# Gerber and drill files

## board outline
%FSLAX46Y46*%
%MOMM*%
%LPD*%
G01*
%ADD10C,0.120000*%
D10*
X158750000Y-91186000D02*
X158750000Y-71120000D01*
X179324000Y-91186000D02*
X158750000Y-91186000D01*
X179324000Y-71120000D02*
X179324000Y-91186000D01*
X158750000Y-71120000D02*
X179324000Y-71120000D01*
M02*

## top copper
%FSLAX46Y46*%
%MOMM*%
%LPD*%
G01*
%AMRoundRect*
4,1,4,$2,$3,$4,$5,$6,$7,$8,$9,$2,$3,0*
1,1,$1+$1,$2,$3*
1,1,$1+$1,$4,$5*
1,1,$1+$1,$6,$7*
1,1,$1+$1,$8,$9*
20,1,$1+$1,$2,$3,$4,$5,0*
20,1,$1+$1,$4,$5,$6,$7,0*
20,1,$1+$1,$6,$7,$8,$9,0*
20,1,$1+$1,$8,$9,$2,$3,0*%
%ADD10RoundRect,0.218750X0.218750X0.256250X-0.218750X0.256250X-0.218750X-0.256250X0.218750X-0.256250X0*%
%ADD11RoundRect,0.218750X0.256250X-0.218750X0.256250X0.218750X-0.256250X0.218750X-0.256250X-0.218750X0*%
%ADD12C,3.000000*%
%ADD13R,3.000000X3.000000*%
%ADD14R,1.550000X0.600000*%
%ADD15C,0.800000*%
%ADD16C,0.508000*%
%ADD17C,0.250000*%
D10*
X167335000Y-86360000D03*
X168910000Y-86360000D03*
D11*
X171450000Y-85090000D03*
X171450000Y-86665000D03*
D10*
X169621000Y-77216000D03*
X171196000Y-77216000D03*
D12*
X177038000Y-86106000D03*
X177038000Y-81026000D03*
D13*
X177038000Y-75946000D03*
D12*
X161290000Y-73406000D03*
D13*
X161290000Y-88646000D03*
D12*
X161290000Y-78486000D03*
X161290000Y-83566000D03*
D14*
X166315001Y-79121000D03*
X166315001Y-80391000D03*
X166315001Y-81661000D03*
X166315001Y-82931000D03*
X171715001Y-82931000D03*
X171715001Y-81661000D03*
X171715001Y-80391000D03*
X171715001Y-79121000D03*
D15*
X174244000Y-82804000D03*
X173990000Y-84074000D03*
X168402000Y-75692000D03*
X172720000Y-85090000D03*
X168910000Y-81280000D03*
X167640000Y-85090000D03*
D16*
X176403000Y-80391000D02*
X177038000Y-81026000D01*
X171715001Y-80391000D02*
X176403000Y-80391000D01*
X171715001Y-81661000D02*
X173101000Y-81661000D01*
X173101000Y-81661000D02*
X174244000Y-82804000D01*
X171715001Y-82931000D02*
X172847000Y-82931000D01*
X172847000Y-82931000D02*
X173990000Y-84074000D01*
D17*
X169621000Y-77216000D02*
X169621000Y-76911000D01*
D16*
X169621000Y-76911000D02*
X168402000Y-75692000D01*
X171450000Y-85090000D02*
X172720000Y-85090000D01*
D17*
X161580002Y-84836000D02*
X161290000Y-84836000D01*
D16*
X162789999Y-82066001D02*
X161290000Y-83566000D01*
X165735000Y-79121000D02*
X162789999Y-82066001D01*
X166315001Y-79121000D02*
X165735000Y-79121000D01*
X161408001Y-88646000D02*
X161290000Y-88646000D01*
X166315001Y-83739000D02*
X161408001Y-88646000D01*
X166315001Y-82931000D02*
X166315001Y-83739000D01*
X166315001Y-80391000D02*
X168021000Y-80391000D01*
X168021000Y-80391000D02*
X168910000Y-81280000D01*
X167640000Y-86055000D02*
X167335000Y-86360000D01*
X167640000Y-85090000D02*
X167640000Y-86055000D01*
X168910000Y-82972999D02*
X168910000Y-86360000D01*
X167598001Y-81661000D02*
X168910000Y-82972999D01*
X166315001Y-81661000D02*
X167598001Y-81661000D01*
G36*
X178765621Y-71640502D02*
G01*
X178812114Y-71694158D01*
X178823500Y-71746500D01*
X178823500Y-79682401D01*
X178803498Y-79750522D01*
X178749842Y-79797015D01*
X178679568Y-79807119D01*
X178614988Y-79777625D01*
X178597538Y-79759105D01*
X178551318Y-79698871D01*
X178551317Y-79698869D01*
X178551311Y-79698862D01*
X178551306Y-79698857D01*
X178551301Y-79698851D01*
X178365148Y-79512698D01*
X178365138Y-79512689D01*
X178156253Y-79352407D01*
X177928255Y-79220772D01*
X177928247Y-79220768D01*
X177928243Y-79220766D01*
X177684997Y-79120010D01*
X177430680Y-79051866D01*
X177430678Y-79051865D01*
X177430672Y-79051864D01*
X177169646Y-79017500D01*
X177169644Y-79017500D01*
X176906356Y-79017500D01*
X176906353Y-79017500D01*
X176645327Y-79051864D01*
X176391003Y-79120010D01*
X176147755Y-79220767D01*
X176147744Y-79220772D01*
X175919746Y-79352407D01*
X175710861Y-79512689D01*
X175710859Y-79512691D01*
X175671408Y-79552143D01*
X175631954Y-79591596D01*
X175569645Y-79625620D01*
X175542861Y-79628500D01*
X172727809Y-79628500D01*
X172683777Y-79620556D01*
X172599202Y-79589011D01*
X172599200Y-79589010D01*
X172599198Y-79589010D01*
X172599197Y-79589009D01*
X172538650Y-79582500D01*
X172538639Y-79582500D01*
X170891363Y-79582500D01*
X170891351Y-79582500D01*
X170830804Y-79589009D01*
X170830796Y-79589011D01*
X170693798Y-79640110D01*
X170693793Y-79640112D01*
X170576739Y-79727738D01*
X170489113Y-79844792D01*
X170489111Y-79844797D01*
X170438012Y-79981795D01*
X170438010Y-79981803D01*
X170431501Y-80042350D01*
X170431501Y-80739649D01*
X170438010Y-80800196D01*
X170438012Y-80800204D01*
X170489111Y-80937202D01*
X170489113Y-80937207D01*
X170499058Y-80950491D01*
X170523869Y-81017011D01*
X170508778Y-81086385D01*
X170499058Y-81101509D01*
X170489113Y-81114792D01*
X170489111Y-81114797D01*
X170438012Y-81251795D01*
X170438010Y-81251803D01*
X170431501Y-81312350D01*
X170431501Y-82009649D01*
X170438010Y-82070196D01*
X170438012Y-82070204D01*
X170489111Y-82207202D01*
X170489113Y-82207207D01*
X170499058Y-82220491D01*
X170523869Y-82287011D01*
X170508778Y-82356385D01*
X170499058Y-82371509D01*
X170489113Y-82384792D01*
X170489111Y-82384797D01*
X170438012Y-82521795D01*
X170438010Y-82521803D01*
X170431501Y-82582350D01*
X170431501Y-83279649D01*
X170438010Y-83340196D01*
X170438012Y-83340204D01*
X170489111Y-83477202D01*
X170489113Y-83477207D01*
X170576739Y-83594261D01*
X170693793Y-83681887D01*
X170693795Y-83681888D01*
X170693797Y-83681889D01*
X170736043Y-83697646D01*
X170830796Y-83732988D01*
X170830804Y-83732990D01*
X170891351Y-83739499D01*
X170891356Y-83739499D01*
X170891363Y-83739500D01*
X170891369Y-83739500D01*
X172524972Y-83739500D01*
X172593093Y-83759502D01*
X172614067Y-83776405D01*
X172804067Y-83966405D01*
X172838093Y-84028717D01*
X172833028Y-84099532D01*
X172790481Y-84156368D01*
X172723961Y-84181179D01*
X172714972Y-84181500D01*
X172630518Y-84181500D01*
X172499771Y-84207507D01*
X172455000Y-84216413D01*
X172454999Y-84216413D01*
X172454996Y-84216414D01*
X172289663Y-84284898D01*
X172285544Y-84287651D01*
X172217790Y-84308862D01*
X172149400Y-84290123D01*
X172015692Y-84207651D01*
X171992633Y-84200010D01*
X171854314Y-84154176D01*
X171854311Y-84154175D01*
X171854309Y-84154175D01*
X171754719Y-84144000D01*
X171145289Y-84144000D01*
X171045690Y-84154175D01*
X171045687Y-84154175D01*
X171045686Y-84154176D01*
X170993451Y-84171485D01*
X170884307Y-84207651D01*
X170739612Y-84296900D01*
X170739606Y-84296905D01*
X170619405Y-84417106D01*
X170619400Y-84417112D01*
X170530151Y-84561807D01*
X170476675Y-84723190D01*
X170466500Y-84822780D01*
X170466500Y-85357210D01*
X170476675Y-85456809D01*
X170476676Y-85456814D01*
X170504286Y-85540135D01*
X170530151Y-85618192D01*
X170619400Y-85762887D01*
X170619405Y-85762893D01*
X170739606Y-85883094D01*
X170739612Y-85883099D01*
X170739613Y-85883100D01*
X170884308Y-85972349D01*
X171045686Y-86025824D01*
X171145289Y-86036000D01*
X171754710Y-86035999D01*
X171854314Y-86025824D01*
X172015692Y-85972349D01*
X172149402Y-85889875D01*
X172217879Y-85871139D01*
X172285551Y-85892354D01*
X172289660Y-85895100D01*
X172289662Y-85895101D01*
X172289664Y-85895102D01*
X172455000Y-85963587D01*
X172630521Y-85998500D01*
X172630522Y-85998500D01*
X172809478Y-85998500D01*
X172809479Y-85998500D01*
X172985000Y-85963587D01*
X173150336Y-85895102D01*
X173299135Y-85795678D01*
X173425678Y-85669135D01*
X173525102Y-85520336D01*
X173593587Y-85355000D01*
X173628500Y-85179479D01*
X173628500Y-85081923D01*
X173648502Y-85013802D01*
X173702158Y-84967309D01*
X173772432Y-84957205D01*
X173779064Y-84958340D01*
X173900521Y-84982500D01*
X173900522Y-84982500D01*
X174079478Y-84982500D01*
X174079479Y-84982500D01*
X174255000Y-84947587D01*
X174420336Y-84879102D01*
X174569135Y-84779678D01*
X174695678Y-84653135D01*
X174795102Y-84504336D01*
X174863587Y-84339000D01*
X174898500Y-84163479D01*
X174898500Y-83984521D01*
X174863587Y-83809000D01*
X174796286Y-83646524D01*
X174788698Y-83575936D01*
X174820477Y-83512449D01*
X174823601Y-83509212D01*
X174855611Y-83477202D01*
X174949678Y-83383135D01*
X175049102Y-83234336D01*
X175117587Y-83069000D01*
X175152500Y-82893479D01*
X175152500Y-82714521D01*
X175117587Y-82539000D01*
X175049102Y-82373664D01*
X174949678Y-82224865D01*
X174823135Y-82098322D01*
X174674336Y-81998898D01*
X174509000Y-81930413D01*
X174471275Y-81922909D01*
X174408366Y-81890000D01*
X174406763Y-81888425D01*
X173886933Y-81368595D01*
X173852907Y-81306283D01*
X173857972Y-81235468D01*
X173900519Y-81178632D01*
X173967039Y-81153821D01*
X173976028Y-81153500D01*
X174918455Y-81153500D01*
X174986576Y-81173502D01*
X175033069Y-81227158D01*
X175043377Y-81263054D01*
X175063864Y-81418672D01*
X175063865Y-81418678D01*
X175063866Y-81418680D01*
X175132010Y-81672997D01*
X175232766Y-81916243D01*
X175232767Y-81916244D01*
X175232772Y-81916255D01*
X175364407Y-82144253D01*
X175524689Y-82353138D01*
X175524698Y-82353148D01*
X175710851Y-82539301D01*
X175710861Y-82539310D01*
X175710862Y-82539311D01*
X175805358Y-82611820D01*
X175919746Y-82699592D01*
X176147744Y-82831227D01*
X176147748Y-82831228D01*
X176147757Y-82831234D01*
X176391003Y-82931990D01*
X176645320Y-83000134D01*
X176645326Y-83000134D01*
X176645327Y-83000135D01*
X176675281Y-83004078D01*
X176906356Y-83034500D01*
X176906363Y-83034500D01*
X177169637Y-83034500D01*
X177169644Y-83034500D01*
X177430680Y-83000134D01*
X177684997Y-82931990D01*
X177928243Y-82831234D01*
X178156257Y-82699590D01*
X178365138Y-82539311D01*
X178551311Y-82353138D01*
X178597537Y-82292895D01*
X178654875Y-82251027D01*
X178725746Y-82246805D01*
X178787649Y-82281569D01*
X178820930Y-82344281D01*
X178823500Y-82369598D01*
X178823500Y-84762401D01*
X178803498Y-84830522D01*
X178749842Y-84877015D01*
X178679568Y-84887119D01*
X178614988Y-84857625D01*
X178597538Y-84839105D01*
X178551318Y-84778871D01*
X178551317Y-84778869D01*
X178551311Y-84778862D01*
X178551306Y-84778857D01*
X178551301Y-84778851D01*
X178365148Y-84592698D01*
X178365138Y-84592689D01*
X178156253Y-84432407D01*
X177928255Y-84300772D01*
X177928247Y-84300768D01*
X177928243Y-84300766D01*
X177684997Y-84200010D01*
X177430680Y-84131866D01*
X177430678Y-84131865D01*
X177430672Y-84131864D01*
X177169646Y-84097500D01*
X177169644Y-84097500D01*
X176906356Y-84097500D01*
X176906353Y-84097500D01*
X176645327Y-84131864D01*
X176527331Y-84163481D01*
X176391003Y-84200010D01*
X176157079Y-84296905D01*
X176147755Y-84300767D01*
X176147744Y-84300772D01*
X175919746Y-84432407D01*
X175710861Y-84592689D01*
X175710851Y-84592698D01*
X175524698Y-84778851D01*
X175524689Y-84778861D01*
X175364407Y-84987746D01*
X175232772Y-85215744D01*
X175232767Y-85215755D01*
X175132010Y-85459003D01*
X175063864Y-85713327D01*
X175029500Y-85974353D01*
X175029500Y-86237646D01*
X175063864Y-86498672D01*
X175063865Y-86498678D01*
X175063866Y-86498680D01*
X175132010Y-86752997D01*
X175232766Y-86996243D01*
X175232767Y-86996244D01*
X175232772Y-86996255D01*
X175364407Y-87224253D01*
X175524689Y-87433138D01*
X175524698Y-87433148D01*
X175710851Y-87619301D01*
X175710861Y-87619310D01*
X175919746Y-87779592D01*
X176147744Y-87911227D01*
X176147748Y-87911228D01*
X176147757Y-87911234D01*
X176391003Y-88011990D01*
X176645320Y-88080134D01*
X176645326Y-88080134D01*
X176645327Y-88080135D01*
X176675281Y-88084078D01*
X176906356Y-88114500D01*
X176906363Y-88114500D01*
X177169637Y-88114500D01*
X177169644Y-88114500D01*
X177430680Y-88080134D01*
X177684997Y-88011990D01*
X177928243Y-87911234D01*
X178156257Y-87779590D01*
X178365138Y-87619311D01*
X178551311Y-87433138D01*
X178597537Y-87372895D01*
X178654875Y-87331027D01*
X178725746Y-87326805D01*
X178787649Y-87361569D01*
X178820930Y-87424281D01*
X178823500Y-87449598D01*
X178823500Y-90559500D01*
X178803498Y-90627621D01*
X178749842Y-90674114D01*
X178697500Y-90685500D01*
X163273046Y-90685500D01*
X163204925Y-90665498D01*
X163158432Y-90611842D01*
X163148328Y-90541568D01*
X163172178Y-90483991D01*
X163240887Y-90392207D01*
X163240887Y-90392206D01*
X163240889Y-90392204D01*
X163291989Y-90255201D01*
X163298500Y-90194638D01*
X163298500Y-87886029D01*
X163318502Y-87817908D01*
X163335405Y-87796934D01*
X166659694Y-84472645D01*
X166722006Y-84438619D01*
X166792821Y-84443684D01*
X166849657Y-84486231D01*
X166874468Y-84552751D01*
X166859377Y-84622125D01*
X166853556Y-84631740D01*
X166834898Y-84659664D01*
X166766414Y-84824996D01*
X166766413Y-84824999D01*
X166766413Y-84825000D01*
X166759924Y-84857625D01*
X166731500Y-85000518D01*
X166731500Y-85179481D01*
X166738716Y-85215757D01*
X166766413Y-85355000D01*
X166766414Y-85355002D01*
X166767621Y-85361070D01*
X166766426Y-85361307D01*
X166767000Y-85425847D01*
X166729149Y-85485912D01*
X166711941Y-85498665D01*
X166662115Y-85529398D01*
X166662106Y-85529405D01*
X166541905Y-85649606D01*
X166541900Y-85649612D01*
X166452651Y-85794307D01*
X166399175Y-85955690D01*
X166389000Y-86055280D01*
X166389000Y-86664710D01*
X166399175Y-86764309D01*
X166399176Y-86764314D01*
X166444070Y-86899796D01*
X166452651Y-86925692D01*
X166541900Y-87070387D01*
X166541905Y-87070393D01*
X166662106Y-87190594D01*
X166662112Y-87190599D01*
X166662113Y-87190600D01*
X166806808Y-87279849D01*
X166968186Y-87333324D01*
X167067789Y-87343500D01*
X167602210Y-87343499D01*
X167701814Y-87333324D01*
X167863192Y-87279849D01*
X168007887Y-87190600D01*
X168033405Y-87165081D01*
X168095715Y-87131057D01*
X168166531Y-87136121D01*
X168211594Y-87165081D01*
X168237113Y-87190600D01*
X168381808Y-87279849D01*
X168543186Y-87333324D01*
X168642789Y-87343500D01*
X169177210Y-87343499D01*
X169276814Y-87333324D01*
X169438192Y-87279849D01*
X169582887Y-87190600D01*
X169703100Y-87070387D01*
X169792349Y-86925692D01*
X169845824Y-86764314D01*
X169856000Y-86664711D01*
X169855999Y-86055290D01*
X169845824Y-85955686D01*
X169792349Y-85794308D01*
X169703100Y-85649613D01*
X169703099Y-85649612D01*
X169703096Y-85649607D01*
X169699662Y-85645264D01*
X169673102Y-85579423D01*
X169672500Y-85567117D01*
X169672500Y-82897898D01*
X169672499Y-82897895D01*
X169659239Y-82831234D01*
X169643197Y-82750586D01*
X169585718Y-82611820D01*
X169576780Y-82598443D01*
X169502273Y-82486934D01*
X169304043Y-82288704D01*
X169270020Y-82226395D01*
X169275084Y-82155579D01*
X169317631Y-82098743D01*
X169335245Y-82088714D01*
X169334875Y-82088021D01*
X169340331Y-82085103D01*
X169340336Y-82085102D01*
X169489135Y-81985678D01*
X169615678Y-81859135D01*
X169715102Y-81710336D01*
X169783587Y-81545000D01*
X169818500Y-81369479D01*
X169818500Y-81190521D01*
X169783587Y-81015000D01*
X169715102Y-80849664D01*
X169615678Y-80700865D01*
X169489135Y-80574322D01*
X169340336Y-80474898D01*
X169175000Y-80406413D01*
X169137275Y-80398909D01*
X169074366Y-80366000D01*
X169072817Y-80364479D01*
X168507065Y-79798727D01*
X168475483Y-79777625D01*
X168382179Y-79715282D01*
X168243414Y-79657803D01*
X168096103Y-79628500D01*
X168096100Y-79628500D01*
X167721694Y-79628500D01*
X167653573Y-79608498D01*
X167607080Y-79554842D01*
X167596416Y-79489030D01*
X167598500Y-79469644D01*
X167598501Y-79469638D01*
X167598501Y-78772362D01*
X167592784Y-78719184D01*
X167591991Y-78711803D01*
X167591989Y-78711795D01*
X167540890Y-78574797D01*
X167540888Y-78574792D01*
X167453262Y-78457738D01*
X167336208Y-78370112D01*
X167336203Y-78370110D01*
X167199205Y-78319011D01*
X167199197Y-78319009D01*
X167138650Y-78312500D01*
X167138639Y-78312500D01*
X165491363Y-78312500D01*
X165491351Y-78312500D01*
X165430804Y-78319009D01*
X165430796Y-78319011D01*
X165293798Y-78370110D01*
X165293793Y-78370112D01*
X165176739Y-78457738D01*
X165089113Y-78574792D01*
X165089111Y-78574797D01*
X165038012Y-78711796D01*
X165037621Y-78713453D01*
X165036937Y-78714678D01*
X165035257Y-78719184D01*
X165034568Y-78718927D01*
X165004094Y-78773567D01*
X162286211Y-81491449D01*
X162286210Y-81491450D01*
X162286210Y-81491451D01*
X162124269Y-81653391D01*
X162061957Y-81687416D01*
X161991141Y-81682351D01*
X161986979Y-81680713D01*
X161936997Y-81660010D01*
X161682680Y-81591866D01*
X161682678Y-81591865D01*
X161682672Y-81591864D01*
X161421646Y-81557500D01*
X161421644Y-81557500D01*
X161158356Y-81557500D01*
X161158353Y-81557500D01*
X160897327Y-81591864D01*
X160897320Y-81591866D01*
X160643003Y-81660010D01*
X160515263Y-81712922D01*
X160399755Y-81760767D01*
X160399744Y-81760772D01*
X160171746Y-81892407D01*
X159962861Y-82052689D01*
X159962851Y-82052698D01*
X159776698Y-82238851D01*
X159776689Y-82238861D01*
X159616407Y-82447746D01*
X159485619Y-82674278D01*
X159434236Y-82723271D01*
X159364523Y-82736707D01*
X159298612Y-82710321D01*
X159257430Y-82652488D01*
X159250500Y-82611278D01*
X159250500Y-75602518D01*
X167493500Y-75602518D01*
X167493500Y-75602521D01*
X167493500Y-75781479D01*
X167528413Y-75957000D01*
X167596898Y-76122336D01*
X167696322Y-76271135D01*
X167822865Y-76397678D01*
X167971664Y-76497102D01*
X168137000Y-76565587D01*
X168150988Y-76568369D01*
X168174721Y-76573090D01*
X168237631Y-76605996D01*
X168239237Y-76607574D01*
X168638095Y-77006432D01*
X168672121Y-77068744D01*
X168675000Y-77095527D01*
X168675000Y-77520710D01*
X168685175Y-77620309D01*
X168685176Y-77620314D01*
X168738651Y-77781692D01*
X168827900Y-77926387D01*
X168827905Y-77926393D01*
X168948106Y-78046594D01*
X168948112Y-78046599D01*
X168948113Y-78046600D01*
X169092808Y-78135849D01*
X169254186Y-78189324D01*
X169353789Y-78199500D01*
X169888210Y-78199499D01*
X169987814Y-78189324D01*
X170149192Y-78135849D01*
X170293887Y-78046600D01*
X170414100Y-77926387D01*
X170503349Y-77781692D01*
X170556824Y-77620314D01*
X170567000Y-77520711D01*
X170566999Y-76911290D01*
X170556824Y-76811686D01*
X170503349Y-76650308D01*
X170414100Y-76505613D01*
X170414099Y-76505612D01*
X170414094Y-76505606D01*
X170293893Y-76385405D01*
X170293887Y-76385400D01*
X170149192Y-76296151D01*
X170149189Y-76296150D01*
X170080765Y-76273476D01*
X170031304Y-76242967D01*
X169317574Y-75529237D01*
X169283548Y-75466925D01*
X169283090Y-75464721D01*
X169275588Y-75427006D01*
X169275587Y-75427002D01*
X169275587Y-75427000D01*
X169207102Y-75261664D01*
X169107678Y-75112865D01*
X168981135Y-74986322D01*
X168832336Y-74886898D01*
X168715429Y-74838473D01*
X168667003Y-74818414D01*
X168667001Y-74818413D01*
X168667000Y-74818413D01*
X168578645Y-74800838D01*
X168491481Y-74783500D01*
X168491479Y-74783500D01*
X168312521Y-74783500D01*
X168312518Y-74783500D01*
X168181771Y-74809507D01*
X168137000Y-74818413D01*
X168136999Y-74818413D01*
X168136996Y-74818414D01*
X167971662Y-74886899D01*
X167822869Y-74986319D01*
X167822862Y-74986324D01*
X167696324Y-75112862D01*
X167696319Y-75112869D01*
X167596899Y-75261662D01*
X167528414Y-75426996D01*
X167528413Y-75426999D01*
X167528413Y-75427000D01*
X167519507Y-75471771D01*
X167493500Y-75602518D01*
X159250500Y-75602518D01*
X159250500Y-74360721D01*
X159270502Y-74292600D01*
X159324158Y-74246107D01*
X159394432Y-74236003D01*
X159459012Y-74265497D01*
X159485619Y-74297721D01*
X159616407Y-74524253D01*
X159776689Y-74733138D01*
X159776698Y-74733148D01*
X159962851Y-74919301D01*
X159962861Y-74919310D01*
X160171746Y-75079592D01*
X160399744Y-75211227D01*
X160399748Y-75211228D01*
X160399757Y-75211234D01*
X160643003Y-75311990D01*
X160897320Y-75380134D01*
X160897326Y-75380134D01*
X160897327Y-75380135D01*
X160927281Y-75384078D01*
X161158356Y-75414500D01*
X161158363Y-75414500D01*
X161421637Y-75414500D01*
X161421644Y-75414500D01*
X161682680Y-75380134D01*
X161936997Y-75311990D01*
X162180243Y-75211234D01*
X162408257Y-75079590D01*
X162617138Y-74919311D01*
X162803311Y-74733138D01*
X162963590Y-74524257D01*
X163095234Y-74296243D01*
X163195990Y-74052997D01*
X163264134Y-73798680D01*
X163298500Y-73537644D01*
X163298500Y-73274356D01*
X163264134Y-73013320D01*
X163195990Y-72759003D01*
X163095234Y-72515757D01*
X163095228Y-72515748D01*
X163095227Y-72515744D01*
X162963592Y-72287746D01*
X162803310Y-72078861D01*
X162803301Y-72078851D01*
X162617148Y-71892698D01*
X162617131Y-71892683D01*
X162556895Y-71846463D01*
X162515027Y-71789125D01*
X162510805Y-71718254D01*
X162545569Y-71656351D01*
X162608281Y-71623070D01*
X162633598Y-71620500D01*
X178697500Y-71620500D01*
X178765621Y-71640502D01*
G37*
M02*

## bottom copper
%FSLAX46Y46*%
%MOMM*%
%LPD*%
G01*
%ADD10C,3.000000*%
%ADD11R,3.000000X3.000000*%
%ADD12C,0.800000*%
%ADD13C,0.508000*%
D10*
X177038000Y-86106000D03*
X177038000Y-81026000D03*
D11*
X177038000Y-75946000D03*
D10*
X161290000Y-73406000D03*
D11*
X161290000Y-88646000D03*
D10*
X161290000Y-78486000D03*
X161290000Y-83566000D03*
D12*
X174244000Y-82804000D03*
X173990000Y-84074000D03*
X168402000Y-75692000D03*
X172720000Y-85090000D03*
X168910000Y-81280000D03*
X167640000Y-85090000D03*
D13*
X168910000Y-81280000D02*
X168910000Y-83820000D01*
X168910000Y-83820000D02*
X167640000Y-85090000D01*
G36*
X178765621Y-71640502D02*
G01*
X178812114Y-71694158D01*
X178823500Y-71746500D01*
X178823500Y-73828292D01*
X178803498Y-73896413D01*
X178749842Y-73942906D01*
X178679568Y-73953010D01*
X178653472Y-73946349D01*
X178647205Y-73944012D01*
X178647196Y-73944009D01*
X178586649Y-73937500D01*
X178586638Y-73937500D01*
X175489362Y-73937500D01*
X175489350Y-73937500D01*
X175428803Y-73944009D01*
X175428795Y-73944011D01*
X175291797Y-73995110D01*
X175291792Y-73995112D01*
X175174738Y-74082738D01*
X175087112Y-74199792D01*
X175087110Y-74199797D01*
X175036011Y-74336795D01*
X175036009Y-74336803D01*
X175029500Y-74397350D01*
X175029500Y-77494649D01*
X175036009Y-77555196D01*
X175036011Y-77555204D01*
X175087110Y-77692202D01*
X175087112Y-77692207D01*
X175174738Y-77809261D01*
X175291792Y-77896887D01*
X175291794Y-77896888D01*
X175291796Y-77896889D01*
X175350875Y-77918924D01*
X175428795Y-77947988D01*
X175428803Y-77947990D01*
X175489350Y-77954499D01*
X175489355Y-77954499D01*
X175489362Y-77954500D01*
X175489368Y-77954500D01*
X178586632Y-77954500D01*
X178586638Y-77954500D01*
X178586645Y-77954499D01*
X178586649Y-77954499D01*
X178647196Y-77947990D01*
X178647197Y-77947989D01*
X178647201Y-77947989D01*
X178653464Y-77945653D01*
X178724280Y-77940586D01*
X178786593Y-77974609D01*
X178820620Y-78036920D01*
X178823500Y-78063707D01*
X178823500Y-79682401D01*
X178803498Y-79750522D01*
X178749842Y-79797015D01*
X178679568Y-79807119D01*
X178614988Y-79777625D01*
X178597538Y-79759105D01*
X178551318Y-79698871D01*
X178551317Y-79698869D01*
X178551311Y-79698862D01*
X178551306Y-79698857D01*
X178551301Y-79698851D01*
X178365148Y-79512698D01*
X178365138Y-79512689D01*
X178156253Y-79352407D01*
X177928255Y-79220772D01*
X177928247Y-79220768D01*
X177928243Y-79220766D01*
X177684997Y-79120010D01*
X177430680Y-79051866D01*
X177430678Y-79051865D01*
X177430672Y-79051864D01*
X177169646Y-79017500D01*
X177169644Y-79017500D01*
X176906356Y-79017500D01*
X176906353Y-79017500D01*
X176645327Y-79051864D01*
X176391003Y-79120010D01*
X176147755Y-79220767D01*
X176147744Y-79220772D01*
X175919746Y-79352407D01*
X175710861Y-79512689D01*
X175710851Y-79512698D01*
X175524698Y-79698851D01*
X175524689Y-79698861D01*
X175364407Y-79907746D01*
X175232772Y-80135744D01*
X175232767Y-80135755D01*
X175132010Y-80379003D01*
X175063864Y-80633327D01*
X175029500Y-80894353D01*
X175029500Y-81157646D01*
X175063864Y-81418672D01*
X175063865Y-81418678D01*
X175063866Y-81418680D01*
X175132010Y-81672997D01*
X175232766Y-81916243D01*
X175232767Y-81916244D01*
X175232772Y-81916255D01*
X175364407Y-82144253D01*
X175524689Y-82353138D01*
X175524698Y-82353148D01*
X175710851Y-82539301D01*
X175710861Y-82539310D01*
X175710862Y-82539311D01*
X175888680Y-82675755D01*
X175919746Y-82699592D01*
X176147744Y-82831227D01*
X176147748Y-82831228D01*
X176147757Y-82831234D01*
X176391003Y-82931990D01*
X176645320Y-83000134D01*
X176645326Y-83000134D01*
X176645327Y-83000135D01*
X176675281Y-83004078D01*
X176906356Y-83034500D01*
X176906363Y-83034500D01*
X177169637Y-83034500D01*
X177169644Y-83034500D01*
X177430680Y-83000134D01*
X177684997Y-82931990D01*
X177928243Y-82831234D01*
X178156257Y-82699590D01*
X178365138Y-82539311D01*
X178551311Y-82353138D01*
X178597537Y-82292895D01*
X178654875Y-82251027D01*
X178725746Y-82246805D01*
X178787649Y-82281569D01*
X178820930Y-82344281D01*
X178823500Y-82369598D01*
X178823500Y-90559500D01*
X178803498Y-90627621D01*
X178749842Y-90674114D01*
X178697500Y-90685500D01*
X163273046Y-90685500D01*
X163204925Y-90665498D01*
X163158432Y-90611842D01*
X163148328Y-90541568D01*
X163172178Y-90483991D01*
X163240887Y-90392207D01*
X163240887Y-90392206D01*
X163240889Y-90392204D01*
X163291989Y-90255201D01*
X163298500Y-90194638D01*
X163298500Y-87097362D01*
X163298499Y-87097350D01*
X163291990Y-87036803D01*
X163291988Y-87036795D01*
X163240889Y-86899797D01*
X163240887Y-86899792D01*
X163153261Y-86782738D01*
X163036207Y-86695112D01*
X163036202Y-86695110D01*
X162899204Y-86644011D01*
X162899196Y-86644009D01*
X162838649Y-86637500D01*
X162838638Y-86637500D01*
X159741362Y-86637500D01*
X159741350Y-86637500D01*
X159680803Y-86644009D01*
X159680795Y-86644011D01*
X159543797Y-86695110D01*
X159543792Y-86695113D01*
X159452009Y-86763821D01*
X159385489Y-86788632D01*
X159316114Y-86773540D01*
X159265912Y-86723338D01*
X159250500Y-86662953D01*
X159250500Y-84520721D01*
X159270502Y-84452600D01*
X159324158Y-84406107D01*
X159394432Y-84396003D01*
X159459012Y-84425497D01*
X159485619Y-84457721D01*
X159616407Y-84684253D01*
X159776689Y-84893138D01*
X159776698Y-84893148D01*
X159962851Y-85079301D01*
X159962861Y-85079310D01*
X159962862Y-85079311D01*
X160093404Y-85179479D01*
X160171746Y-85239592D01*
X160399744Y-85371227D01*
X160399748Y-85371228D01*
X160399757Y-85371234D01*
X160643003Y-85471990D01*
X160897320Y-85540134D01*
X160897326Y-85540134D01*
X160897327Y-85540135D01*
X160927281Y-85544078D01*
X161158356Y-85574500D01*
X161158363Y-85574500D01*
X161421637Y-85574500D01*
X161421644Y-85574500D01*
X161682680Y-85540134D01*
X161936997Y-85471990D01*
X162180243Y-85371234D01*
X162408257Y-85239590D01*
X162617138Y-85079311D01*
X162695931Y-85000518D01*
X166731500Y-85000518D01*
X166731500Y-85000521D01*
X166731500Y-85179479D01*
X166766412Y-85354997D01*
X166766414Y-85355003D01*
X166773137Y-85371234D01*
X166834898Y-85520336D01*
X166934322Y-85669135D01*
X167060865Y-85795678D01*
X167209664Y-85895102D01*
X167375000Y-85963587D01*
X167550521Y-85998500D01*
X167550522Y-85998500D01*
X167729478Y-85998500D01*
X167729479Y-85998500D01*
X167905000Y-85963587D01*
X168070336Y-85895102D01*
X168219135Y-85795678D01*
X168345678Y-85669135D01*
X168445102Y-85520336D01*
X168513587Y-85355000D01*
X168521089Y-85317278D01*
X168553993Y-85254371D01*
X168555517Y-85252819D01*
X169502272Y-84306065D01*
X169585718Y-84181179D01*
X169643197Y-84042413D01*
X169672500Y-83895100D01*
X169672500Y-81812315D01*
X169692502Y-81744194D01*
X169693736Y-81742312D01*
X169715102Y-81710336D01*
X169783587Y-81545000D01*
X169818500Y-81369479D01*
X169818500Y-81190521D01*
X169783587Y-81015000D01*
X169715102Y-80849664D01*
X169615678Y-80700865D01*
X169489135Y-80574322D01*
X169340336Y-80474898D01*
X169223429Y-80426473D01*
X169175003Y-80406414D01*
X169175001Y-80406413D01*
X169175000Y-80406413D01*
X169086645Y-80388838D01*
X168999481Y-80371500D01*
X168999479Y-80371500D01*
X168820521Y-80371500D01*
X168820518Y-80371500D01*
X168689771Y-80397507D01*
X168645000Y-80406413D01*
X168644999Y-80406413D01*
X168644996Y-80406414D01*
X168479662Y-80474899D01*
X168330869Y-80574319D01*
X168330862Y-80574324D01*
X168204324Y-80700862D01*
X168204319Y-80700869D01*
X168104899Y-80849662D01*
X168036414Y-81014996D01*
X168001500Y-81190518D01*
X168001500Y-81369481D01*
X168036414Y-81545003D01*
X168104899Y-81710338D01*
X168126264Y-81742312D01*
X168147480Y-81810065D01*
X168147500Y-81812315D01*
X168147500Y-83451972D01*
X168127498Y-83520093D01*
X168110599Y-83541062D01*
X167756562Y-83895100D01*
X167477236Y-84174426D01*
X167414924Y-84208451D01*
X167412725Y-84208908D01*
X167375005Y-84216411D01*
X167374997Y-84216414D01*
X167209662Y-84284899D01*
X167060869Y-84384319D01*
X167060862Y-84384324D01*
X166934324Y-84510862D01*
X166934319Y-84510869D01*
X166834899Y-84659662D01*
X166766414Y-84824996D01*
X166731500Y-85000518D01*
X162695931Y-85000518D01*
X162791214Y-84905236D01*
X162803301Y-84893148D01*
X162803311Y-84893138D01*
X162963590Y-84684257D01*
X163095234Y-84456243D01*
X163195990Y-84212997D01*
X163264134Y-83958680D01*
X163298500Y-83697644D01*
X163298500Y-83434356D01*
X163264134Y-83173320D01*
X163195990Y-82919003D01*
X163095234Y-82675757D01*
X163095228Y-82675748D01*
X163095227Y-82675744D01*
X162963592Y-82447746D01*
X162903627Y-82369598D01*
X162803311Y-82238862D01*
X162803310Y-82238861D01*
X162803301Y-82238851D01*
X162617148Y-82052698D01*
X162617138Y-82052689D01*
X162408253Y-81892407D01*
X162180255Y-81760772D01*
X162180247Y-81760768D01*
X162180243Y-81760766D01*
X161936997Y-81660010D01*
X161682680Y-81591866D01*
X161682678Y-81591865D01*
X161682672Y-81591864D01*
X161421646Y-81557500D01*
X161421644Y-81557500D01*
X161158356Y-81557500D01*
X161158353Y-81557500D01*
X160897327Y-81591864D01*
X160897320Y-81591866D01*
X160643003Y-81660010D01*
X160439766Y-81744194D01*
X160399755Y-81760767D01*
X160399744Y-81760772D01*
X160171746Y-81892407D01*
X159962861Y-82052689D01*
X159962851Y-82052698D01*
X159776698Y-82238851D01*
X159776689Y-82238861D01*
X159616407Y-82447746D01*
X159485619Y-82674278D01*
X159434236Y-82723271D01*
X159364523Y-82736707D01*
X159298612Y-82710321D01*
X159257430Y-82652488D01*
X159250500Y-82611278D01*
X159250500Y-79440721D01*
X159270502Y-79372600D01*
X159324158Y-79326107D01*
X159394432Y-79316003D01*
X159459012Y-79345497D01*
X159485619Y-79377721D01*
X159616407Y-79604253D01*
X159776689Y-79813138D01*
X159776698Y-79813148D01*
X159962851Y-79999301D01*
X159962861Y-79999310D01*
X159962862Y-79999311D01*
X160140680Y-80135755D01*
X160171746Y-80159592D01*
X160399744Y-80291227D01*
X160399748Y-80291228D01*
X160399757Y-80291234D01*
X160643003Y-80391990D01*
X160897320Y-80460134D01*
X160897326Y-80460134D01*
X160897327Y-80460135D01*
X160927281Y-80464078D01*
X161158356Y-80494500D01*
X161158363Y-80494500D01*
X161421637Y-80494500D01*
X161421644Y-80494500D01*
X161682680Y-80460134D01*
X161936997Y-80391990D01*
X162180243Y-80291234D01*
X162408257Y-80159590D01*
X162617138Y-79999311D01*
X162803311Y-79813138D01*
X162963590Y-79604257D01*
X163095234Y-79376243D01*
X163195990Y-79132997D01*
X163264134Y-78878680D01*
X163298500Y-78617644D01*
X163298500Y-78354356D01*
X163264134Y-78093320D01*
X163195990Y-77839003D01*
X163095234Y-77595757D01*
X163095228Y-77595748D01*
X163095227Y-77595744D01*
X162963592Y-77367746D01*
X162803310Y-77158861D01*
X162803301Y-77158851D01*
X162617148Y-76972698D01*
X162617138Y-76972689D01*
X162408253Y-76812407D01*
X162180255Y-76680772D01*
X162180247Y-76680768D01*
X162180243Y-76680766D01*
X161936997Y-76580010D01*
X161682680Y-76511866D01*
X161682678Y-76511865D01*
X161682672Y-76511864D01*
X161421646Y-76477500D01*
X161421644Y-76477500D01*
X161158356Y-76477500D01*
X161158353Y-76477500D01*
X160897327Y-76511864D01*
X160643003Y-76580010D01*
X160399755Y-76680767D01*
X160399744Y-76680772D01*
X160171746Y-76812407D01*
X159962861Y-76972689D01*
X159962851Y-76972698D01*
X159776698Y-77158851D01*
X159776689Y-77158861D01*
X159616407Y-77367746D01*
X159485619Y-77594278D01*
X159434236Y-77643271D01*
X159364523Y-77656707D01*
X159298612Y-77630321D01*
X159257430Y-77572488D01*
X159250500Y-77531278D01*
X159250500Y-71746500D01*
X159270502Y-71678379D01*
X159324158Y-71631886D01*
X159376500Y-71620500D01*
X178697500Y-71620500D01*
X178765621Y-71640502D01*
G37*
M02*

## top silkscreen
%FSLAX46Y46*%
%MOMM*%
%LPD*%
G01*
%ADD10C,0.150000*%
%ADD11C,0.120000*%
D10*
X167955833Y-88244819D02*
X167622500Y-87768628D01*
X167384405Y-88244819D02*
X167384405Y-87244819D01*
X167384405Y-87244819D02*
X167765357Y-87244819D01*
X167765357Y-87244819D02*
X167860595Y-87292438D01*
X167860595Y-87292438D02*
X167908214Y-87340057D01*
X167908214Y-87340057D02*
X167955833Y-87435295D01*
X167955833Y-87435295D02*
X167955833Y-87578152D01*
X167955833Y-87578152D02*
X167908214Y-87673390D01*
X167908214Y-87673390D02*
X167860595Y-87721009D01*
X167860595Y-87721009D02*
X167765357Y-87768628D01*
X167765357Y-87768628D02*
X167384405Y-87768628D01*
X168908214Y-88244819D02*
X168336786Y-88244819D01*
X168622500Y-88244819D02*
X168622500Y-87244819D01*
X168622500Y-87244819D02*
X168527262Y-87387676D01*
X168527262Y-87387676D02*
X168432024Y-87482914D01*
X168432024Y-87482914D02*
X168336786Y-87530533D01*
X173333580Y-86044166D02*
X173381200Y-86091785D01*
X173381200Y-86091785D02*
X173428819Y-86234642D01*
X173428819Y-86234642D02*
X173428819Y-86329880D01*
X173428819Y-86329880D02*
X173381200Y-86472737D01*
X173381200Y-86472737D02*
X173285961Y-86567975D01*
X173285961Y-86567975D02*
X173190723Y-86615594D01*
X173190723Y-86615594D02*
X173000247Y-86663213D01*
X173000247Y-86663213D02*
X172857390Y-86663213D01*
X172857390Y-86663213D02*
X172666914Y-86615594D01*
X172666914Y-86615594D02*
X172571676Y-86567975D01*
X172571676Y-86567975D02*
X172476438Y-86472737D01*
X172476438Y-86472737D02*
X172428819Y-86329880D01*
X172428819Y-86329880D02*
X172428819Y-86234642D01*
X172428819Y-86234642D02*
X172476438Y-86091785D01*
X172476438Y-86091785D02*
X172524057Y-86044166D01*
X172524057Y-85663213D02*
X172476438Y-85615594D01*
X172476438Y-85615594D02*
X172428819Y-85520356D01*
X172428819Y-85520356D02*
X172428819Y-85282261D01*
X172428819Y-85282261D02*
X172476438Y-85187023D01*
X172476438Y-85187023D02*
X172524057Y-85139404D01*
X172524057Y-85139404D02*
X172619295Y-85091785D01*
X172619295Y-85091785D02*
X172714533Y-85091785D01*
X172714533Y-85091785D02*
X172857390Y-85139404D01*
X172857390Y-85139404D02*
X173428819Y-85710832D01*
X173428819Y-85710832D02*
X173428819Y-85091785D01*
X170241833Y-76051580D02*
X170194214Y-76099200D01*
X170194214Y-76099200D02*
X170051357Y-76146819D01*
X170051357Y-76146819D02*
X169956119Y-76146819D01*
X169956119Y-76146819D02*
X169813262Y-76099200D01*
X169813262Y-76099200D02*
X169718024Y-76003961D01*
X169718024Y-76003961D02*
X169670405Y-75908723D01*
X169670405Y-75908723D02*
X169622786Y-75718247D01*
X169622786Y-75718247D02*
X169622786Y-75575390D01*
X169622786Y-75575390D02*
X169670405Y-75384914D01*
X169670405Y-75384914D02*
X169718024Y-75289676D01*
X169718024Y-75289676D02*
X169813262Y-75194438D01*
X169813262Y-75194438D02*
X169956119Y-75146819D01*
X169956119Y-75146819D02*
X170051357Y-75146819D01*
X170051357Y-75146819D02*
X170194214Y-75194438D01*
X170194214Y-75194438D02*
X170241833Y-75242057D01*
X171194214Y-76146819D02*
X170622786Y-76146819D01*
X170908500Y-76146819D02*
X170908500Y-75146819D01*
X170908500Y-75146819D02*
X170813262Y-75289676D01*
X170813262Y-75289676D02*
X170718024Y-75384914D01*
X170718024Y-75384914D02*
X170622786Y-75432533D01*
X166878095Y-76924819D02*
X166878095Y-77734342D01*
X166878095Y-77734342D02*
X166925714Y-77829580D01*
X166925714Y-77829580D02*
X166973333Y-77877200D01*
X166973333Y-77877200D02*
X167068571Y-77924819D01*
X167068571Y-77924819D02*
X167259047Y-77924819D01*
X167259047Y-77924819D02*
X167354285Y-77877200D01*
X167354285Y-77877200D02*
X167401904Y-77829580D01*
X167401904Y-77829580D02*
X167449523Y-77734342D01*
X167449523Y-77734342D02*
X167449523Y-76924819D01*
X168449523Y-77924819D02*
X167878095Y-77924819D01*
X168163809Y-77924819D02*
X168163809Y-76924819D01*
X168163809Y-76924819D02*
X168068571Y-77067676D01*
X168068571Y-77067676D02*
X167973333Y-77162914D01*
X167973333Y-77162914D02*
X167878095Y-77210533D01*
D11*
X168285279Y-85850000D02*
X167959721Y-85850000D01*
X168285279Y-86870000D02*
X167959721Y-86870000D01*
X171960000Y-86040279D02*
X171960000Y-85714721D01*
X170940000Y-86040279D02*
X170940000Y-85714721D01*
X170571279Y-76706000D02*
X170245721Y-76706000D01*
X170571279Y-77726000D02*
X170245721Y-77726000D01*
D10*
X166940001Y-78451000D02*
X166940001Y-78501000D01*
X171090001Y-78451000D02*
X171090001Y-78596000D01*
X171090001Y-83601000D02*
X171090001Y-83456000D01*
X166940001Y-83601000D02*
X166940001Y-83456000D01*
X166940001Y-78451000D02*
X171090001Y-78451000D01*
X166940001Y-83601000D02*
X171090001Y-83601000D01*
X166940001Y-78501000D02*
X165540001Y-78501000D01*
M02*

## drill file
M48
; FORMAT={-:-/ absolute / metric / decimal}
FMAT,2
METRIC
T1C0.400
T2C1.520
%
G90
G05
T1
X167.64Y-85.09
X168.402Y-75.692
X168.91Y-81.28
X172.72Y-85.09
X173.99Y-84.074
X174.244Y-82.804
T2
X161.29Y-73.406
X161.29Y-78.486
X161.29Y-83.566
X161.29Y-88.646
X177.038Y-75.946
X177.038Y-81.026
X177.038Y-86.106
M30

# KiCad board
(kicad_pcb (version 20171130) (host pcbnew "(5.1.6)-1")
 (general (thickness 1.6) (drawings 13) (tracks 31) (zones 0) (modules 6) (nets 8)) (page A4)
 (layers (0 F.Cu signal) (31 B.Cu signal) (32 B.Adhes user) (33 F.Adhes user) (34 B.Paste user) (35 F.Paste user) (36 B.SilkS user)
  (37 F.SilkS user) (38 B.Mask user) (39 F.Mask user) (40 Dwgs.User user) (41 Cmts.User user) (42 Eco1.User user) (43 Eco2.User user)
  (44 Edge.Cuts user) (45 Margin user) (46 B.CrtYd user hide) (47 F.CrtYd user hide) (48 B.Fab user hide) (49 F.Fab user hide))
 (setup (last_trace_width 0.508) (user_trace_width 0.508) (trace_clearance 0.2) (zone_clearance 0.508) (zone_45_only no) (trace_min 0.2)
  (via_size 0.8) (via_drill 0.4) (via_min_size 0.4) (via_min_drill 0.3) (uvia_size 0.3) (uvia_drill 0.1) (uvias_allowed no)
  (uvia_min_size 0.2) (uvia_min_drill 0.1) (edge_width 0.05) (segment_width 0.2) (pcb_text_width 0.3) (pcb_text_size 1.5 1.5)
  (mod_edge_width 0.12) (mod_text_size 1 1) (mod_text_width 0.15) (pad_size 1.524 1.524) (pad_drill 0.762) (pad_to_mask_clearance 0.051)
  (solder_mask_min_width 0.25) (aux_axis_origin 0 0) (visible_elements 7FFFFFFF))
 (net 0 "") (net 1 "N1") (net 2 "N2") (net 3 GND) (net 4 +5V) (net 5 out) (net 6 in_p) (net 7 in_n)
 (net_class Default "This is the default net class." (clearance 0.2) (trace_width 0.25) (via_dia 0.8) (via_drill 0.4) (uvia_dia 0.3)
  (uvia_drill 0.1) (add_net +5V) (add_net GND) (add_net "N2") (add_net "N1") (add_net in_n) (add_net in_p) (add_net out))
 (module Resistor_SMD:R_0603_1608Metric (layer F.Cu) (at 168.1225 86.36 180)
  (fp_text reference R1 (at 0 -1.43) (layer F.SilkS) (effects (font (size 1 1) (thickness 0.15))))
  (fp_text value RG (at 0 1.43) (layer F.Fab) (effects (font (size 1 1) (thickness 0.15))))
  (fp_line (start -0.162779 0.51) (end 0.162779 0.51) (layer F.SilkS) (width 0.12))
  (fp_line (start -0.162779 -0.51) (end 0.162779 -0.51) (layer F.SilkS) (width 0.12))
  (pad 2 smd roundrect (at 0.7875 0 180) (size 0.875 0.95) (layers F.Cu F.Paste F.Mask) (roundrect_rratio 0.25) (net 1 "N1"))
  (pad 1 smd roundrect (at -0.7875 0 180) (size 0.875 0.95) (layers F.Cu F.Paste F.Mask) (roundrect_rratio 0.25) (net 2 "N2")))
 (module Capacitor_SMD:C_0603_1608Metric (layer F.Cu) (at 171.45 85.8775 90)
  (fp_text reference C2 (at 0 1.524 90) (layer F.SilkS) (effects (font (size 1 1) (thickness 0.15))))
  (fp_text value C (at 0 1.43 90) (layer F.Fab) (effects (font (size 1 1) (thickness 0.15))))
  (fp_line (start -0.162779 0.51) (end 0.162779 0.51) (layer F.SilkS) (width 0.12))
  (fp_line (start -0.162779 -0.51) (end 0.162779 -0.51) (layer F.SilkS) (width 0.12))
  (pad 2 smd roundrect (at 0.7875 0 90) (size 0.875 0.95) (layers F.Cu F.Paste F.Mask) (roundrect_rratio 0.25) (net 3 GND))
  (pad 1 smd roundrect (at -0.7875 0 90) (size 0.875 0.95) (layers F.Cu F.Paste F.Mask) (roundrect_rratio 0.25) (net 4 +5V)))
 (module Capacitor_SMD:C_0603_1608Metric (layer F.Cu) (at 170.4085 77.216 180)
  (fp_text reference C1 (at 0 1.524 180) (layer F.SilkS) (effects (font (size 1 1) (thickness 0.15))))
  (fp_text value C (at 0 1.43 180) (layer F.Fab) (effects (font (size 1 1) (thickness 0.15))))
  (fp_line (start -0.162779 0.51) (end 0.162779 0.51) (layer F.SilkS) (width 0.12))
  (fp_line (start -0.162779 -0.51) (end 0.162779 -0.51) (layer F.SilkS) (width 0.12))
  (pad 2 smd roundrect (at 0.7875 0 180) (size 0.875 0.95) (layers F.Cu F.Paste F.Mask) (roundrect_rratio 0.25) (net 3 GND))
  (pad 1 smd roundrect (at -0.7875 0 180) (size 0.875 0.95) (layers F.Cu F.Paste F.Mask) (roundrect_rratio 0.25) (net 4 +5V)))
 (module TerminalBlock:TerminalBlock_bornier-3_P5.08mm (layer F.Cu) (at 177.038 75.946 270)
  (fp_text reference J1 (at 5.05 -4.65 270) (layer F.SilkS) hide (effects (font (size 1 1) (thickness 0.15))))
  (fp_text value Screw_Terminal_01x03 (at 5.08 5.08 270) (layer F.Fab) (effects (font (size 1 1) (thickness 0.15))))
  (pad 3 thru_hole circle (at 10.16 0 270) (size 3 3) (drill 1.52) (layers *.Cu *.Mask) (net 3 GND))
  (pad 2 thru_hole circle (at 5.08 0 270) (size 3 3) (drill 1.52) (layers *.Cu *.Mask) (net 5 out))
  (pad 1 thru_hole rect (at 0 0 270) (size 3 3) (drill 1.52) (layers *.Cu *.Mask) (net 4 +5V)))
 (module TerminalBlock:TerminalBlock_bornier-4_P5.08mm (layer F.Cu) (at 161.29 88.646 90)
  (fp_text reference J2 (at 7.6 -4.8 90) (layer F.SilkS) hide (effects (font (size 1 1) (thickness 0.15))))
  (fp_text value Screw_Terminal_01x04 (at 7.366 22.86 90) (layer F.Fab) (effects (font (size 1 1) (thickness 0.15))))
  (pad 4 thru_hole circle (at 15.24 0 90) (size 3 3) (drill 1.52) (layers *.Cu *.Mask) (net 3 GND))
  (pad 1 thru_hole rect (at 0 0 90) (size 3 3) (drill 1.52) (layers *.Cu *.Mask) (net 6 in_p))
  (pad 3 thru_hole circle (at 10.16 0 90) (size 3 3) (drill 1.52) (layers *.Cu *.Mask) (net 4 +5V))
  (pad 2 thru_hole circle (at 5.08 0 90) (size 3 3) (drill 1.52) (layers *.Cu *.Mask) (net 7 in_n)))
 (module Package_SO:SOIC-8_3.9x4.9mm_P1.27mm (layer F.Cu) (at 169.015001 81.026)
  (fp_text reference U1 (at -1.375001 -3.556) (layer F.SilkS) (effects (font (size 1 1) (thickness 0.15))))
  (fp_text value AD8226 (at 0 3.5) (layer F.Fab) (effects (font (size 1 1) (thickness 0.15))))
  (fp_line (start -2.075 -2.575) (end -2.075 -2.525) (layer F.SilkS) (width 0.15))
  (fp_line (start 2.075 -2.575) (end 2.075 -2.43) (layer F.SilkS) (width 0.15))
  (fp_line (start 2.075 2.575) (end 2.075 2.43) (layer F.SilkS) (width 0.15))
  (fp_line (start -2.075 2.575) (end -2.075 2.43) (layer F.SilkS) (width 0.15))
  (fp_line (start -2.075 -2.575) (end 2.075 -2.575) (layer F.SilkS) (width 0.15))
  (fp_line (start -2.075 2.575) (end 2.075 2.575) (layer F.SilkS) (width 0.15))
  (fp_line (start -2.075 -2.525) (end -3.475 -2.525) (layer F.SilkS) (width 0.15))
  (pad 1 smd rect (at -2.7 -1.905) (size 1.55 0.6) (layers F.Cu F.Paste F.Mask) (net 7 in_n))
  (pad 2 smd rect (at -2.7 -0.635) (size 1.55 0.6) (layers F.Cu F.Paste F.Mask) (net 1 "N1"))
  (pad 3 smd rect (at -2.7 0.635) (size 1.55 0.6) (layers F.Cu F.Paste F.Mask) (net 2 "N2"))
  (pad 4 smd rect (at -2.7 1.905) (size 1.55 0.6) (layers F.Cu F.Paste F.Mask) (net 6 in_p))
  (pad 5 smd rect (at 2.7 1.905) (size 1.55 0.6) (layers F.Cu F.Paste F.Mask) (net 3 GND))
  (pad 6 smd rect (at 2.7 0.635) (size 1.55 0.6) (layers F.Cu F.Paste F.Mask) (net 3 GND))
  (pad 7 smd rect (at 2.7 -0.635) (size 1.55 0.6) (layers F.Cu F.Paste F.Mask) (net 5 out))
  (pad 8 smd rect (at 2.7 -1.905) (size 1.55 0.6) (layers F.Cu F.Paste F.Mask) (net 4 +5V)))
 (gr_line (start 158.75 91.186) (end 158.75 71.12) (layer Edge.Cuts) (width 0.12))
 (gr_line (start 179.324 91.186) (end 158.75 91.186) (layer Edge.Cuts) (width 0.12))
 (gr_line (start 179.324 71.12) (end 179.324 91.186) (layer Edge.Cuts) (width 0.12))
 (gr_line (start 158.75 71.12) (end 179.324 71.12) (layer Edge.Cuts) (width 0.12))
 (segment (start 176.403 80.391) (end 177.038 81.026) (width 0.508) (layer F.Cu) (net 5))
 (segment (start 171.715001 80.391) (end 176.403 80.391) (width 0.508) (layer F.Cu) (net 5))
 (via (at 174.244 82.804) (size 0.8) (drill 0.4) (layers F.Cu B.Cu) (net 3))
 (segment (start 171.715001 81.661) (end 173.101 81.661) (width 0.508) (layer F.Cu) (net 3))
 (segment (start 173.101 81.661) (end 174.244 82.804) (width 0.508) (layer F.Cu) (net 3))
 (via (at 173.99 84.074) (size 0.8) (drill 0.4) (layers F.Cu B.Cu) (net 3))
 (segment (start 171.715001 82.931) (end 172.847 82.931) (width 0.508) (layer F.Cu) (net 3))
 (segment (start 172.847 82.931) (end 173.99 84.074) (width 0.508) (layer F.Cu) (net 3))
 (via (at 168.402 75.692) (size 0.8) (drill 0.4) (layers F.Cu B.Cu) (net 3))
 (segment (start 169.621 77.216) (end 169.621 76.911) (width 0.25) (layer F.Cu) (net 3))
 (segment (start 169.621 76.911) (end 168.402 75.692) (width 0.508) (layer F.Cu) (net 3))
 (via (at 172.72 85.09) (size 0.8) (drill 0.4) (layers F.Cu B.Cu) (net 3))
 (segment (start 171.45 85.09) (end 172.72 85.09) (width 0.508) (layer F.Cu) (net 3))
 (segment (start 161.580002 84.836) (end 161.29 84.836) (width 0.25) (layer F.Cu) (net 7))
 (segment (start 162.789999 82.066001) (end 161.29 83.566) (width 0.508) (layer F.Cu) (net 7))
 (segment (start 165.735 79.121) (end 162.789999 82.066001) (width 0.508) (layer F.Cu) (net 7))
 (segment (start 166.315001 79.121) (end 165.735 79.121) (width 0.508) (layer F.Cu) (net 7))
 (segment (start 161.408001 88.646) (end 161.29 88.646) (width 0.508) (layer F.Cu) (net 6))
 (segment (start 166.315001 83.739) (end 161.408001 88.646) (width 0.508) (layer F.Cu) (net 6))
 (segment (start 166.315001 82.931) (end 166.315001 83.739) (width 0.508) (layer F.Cu) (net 6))
 (via (at 168.91 81.28) (size 0.8) (drill 0.4) (layers F.Cu B.Cu) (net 1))
 (segment (start 166.315001 80.391) (end 168.021 80.391) (width 0.508) (layer F.Cu) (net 1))
 (segment (start 168.021 80.391) (end 168.91 81.28) (width 0.508) (layer F.Cu) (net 1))
 (segment (start 168.91 81.28) (end 168.91 83.82) (width 0.508) (layer B.Cu) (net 1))
 (via (at 167.64 85.09) (size 0.8) (drill 0.4) (layers F.Cu B.Cu) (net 1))
 (segment (start 168.91 83.82) (end 167.64 85.09) (width 0.508) (layer B.Cu) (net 1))
 (segment (start 167.64 86.055) (end 167.335 86.36) (width 0.508) (layer F.Cu) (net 1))
 (segment (start 167.64 85.09) (end 167.64 86.055) (width 0.508) (layer F.Cu) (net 1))
 (segment (start 168.91 82.972999) (end 168.91 86.36) (width 0.508) (layer F.Cu) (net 2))
 (segment (start 167.598001 81.661) (end 168.91 82.972999) (width 0.508) (layer F.Cu) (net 2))
 (segment (start 166.315001 81.661) (end 167.598001 81.661) (width 0.508) (layer F.Cu) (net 2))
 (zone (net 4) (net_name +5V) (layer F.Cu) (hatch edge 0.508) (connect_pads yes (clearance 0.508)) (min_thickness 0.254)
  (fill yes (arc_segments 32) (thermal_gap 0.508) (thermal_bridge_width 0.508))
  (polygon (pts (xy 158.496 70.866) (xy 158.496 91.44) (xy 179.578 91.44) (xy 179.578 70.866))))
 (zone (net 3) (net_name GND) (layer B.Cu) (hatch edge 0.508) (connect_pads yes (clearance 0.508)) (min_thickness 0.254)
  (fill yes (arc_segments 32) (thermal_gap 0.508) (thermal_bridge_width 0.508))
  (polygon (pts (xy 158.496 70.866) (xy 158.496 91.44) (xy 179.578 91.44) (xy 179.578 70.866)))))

